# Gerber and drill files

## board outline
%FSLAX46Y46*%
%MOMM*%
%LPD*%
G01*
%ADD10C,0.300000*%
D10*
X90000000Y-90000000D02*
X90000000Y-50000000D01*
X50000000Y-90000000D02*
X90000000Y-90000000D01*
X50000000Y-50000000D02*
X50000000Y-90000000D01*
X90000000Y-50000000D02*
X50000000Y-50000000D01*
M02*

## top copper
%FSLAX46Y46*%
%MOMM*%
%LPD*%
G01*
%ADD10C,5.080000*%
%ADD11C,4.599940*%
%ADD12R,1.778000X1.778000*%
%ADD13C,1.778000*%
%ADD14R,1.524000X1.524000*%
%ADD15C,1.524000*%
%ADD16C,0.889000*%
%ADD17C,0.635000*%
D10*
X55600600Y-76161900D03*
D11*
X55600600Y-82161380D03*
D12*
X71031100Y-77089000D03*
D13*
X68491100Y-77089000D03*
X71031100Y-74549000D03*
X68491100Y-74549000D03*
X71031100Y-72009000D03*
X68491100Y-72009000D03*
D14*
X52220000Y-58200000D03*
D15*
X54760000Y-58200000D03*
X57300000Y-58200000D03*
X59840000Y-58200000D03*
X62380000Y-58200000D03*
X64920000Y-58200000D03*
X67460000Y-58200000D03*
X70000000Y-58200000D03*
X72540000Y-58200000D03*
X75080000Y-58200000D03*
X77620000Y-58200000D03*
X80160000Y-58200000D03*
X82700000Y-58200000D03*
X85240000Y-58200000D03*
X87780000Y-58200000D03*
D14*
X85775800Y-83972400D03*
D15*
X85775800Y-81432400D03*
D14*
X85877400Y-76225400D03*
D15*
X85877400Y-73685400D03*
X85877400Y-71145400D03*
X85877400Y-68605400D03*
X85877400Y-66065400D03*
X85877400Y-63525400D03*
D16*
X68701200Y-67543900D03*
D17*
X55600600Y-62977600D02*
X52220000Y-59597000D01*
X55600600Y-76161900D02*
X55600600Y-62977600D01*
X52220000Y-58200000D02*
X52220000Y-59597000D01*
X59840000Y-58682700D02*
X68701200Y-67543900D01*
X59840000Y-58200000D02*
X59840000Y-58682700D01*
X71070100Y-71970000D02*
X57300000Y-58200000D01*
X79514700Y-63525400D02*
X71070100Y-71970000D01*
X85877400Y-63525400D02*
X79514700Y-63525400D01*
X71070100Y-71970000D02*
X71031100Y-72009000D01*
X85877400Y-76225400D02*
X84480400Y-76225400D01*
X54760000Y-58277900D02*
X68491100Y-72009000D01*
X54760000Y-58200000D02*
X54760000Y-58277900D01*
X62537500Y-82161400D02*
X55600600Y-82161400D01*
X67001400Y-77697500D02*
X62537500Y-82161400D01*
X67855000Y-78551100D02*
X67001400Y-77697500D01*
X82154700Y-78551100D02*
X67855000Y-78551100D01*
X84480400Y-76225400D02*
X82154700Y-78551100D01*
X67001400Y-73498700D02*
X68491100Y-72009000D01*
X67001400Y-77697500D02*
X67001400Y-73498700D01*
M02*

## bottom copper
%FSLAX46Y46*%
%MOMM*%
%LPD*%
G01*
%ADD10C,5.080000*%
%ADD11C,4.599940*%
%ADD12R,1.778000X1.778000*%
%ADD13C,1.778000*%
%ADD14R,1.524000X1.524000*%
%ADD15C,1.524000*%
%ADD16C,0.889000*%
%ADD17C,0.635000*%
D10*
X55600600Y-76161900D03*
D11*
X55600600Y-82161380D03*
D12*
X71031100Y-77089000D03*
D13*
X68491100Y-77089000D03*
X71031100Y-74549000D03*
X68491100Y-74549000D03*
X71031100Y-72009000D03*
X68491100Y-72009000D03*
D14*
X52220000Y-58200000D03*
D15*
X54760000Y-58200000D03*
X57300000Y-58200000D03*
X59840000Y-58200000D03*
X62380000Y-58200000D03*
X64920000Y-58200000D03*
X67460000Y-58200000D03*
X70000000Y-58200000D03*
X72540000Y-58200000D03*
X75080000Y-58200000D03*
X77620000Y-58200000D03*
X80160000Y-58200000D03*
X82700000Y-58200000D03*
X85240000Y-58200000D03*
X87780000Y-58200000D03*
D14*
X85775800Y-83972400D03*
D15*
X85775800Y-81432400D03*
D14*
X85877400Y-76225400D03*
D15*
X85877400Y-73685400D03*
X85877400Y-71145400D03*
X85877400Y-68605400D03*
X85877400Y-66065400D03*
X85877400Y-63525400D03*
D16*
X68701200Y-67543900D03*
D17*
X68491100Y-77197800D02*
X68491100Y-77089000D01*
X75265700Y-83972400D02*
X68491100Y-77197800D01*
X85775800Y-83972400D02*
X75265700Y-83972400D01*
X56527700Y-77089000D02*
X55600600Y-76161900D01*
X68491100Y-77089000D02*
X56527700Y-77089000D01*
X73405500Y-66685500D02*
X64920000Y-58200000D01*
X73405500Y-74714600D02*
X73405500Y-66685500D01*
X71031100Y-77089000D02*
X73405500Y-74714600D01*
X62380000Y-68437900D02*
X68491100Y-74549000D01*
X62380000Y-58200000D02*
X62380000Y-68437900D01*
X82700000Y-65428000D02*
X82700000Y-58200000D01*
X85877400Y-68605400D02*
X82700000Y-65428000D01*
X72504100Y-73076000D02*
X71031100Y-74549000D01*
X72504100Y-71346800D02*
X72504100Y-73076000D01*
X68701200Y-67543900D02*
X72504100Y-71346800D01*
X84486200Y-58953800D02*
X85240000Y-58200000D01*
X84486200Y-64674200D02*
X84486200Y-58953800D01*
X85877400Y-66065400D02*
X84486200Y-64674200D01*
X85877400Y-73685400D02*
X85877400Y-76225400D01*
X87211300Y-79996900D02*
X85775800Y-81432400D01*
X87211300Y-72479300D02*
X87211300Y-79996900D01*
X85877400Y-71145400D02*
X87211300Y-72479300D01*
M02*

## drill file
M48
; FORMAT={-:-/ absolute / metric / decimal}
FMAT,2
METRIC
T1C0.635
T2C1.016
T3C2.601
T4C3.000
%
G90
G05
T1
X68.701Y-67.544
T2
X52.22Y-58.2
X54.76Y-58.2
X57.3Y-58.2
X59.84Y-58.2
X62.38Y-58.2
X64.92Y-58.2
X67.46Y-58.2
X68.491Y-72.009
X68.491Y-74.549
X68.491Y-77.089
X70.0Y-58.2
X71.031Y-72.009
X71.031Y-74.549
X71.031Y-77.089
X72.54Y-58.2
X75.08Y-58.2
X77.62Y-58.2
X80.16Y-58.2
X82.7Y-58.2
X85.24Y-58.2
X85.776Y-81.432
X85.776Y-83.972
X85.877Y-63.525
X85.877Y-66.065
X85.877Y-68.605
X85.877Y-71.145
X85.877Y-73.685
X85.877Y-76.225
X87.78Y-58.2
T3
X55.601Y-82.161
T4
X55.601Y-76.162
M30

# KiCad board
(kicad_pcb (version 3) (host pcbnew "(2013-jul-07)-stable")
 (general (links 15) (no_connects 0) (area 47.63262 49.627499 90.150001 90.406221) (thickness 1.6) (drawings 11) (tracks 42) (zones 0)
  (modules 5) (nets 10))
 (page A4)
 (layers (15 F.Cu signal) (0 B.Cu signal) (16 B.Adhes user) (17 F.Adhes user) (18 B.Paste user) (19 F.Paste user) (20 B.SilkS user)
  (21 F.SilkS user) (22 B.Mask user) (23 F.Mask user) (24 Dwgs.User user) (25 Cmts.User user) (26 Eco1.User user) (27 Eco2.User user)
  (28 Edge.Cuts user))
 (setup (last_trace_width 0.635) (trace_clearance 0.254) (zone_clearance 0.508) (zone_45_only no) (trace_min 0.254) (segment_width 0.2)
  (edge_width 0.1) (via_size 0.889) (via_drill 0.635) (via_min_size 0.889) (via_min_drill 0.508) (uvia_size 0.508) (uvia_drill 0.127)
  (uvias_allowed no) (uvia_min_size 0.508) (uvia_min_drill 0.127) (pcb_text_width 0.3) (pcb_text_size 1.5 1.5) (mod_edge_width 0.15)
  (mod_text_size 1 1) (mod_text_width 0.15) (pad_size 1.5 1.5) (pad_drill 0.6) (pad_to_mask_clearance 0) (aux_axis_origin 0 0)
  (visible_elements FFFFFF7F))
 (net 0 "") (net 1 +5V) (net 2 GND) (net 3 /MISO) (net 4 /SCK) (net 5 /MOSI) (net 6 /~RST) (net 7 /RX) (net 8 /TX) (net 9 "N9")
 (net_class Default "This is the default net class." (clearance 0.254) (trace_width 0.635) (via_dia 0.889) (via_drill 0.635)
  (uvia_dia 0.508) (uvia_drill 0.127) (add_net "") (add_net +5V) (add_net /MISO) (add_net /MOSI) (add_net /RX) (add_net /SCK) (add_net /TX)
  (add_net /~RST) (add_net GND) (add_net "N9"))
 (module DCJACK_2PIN (layer F.Cu) (at 55.6006 76.1619 270)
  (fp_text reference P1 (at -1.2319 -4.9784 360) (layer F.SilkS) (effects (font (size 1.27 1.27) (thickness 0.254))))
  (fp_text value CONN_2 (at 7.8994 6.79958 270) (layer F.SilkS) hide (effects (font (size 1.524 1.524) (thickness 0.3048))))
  (pad 1 thru_hole circle (at 0 0 270) (size 5.08 5.08) (drill 2.99974) (layers *.Cu *.Mask F.SilkS) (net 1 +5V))
  (pad 2 thru_hole circle (at 5.99948 0 270) (size 4.59994 4.59994) (drill 2.60096) (layers *.Cu *.Mask F.SilkS) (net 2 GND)))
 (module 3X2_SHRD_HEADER (layer F.Cu) (at 69.7611 74.549 90)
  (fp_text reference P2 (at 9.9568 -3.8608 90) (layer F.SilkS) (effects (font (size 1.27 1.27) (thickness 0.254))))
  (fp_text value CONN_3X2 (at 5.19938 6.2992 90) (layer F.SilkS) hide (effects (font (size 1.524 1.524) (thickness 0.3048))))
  (pad 1 thru_hole rect (at -2.54 1.27 90) (size 1.778 1.778) (drill 1.016) (layers *.Cu *.Mask F.SilkS) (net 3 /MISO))
  (pad 2 thru_hole circle (at -2.54 -1.27 90) (size 1.778 1.778) (drill 1.016) (layers *.Cu *.Mask F.SilkS) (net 1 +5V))
  (pad 3 thru_hole circle (at 0 1.27 90) (size 1.778 1.778) (drill 1.016) (layers *.Cu *.Mask F.SilkS) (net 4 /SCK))
  (pad 4 thru_hole circle (at 0 -1.27 90) (size 1.778 1.778) (drill 1.016) (layers *.Cu *.Mask F.SilkS) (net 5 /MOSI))
  (pad 5 thru_hole circle (at 2.54 1.27 90) (size 1.778 1.778) (drill 1.016) (layers *.Cu *.Mask F.SilkS) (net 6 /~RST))
  (pad 6 thru_hole circle (at 2.54 -1.27 90) (size 1.778 1.778) (drill 1.016) (layers *.Cu *.Mask F.SilkS) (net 2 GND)))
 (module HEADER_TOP (layer F.Cu) (at 70 58.2)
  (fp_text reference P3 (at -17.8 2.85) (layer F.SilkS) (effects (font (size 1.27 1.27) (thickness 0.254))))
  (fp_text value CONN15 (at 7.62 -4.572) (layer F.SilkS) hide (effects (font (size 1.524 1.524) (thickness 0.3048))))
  (pad 1 thru_hole rect (at -17.78 0) (size 1.524 1.524) (drill 1.016) (layers *.Cu *.Mask F.SilkS) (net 1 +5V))
  (pad 2 thru_hole circle (at -15.24 0) (size 1.524 1.524) (drill 1.016) (layers *.Cu *.Mask F.SilkS) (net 2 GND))
  (pad 3 thru_hole circle (at -12.7 0) (size 1.524 1.524) (drill 1.016) (layers *.Cu *.Mask F.SilkS) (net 6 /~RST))
  (pad 4 thru_hole circle (at -10.16 0) (size 1.524 1.524) (drill 1.016) (layers *.Cu *.Mask F.SilkS) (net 4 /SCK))
  (pad 5 thru_hole circle (at -7.62 0) (size 1.524 1.524) (drill 1.016) (layers *.Cu *.Mask F.SilkS) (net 5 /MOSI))
  (pad 6 thru_hole circle (at -5.08 0) (size 1.524 1.524) (drill 1.016) (layers *.Cu *.Mask F.SilkS) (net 3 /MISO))
  (pad 7 thru_hole circle (at -2.54 0) (size 1.524 1.524) (drill 1.016) (layers *.Cu *.Mask F.SilkS))
  (pad 8 thru_hole circle (at 0 0) (size 1.524 1.524) (drill 1.016) (layers *.Cu *.Mask F.SilkS))
  (pad 9 thru_hole circle (at 2.54 0) (size 1.524 1.524) (drill 1.016) (layers *.Cu *.Mask F.SilkS))
  (pad 10 thru_hole circle (at 5.08 0) (size 1.524 1.524) (drill 1.016) (layers *.Cu *.Mask F.SilkS))
  (pad 11 thru_hole circle (at 7.62 0) (size 1.524 1.524) (drill 1.016) (layers *.Cu *.Mask F.SilkS))
  (pad 12 thru_hole circle (at 10.16 0) (size 1.524 1.524) (drill 1.016) (layers *.Cu *.Mask F.SilkS))
  (pad 13 thru_hole circle (at 12.7 0) (size 1.524 1.524) (drill 1.016) (layers *.Cu *.Mask F.SilkS) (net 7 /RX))
  (pad 14 thru_hole circle (at 15.24 0) (size 1.524 1.524) (drill 1.016) (layers *.Cu *.Mask F.SilkS) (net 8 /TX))
  (pad 15 thru_hole circle (at 17.78 0) (size 1.524 1.524) (drill 1.016) (layers *.Cu *.Mask F.SilkS)))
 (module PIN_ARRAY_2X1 (layer F.Cu) (at 85.7758 82.7024 90)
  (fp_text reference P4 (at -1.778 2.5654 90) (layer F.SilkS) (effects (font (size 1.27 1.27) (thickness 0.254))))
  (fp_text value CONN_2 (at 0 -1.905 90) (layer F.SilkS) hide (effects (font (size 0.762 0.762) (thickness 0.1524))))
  (pad 1 thru_hole rect (at -1.27 0 90) (size 1.524 1.524) (drill 1.016) (layers *.Cu *.Mask F.SilkS) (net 1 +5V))
  (pad 2 thru_hole circle (at 1.27 0 90) (size 1.524 1.524) (drill 1.016) (layers *.Cu *.Mask F.SilkS) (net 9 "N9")))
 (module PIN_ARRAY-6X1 (layer F.Cu) (at 85.8774 69.8754 90)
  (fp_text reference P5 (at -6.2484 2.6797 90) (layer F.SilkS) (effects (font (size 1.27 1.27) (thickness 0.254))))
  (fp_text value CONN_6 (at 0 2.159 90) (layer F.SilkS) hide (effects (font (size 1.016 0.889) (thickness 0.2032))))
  (pad 1 thru_hole rect (at -6.35 0 90) (size 1.524 1.524) (drill 1.016) (layers *.Cu *.Mask F.SilkS) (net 2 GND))
  (pad 2 thru_hole circle (at -3.81 0 90) (size 1.524 1.524) (drill 1.016) (layers *.Cu *.Mask F.SilkS) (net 2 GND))
  (pad 3 thru_hole circle (at -1.27 0 90) (size 1.524 1.524) (drill 1.016) (layers *.Cu *.Mask F.SilkS) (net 9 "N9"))
  (pad 4 thru_hole circle (at 1.27 0 90) (size 1.524 1.524) (drill 1.016) (layers *.Cu *.Mask F.SilkS) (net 7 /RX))
  (pad 5 thru_hole circle (at 3.81 0 90) (size 1.524 1.524) (drill 1.016) (layers *.Cu *.Mask F.SilkS) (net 8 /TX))
  (pad 6 thru_hole circle (at 6.35 0 90) (size 1.524 1.524) (drill 1.016) (layers *.Cu *.Mask F.SilkS) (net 6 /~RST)))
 (gr_line (start 90 90) (end 90 50) (angle 90) (layer Edge.Cuts) (width 0.3))
 (gr_line (start 50 90) (end 90 90) (angle 90) (layer Edge.Cuts) (width 0.3))
 (gr_line (start 50 50) (end 50 90) (angle 90) (layer Edge.Cuts) (width 0.3))
 (gr_line (start 90 50) (end 50 50) (angle 90) (layer Edge.Cuts) (width 0.3))
 (segment (start 55.6006 62.9776) (end 52.22 59.597) (width 0.635) (layer F.Cu) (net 1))
 (segment (start 55.6006 76.1619) (end 55.6006 62.9776) (width 0.635) (layer F.Cu) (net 1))
 (segment (start 52.22 58.2) (end 52.22 59.597) (width 0.635) (layer F.Cu) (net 1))
 (segment (start 68.4911 77.1978) (end 68.4911 77.089) (width 0.635) (layer B.Cu) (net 1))
 (segment (start 75.2657 83.9724) (end 68.4911 77.1978) (width 0.635) (layer B.Cu) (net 1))
 (segment (start 85.7758 83.9724) (end 75.2657 83.9724) (width 0.635) (layer B.Cu) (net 1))
 (segment (start 56.5277 77.089) (end 55.6006 76.1619) (width 0.635) (layer B.Cu) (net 1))
 (segment (start 68.4911 77.089) (end 56.5277 77.089) (width 0.635) (layer B.Cu) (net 1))
 (segment (start 73.4055 66.6855) (end 64.92 58.2) (width 0.635) (layer B.Cu) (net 3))
 (segment (start 73.4055 74.7146) (end 73.4055 66.6855) (width 0.635) (layer B.Cu) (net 3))
 (segment (start 71.0311 77.089) (end 73.4055 74.7146) (width 0.635) (layer B.Cu) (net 3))
 (segment (start 62.38 68.4379) (end 68.4911 74.549) (width 0.635) (layer B.Cu) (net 5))
 (segment (start 62.38 58.2) (end 62.38 68.4379) (width 0.635) (layer B.Cu) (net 5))
 (segment (start 82.7 65.428) (end 82.7 58.2) (width 0.635) (layer B.Cu) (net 7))
 (segment (start 85.8774 68.6054) (end 82.7 65.428) (width 0.635) (layer B.Cu) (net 7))
 (via (at 68.7012 67.5439) (size 0.889) (layers F.Cu B.Cu) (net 4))
 (segment (start 72.5041 73.076) (end 71.0311 74.549) (width 0.635) (layer B.Cu) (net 4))
 (segment (start 72.5041 71.3468) (end 72.5041 73.076) (width 0.635) (layer B.Cu) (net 4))
 (segment (start 68.7012 67.5439) (end 72.5041 71.3468) (width 0.635) (layer B.Cu) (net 4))
 (segment (start 59.84 58.6827) (end 68.7012 67.5439) (width 0.635) (layer F.Cu) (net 4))
 (segment (start 59.84 58.2) (end 59.84 58.6827) (width 0.635) (layer F.Cu) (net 4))
 (segment (start 84.4862 58.9538) (end 85.24 58.2) (width 0.635) (layer B.Cu) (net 8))
 (segment (start 84.4862 64.6742) (end 84.4862 58.9538) (width 0.635) (layer B.Cu) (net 8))
 (segment (start 85.8774 66.0654) (end 84.4862 64.6742) (width 0.635) (layer B.Cu) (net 8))
 (segment (start 71.0701 71.97) (end 57.3 58.2) (width 0.635) (layer F.Cu) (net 6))
 (segment (start 79.5147 63.5254) (end 71.0701 71.97) (width 0.635) (layer F.Cu) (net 6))
 (segment (start 85.8774 63.5254) (end 79.5147 63.5254) (width 0.635) (layer F.Cu) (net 6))
 (segment (start 71.0701 71.97) (end 71.0311 72.009) (width 0.635) (layer F.Cu) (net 6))
 (segment (start 85.8774 73.6854) (end 85.8774 76.2254) (width 0.635) (layer B.Cu) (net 2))
 (segment (start 85.8774 76.2254) (end 84.4804 76.2254) (width 0.635) (layer F.Cu) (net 2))
 (segment (start 54.76 58.2779) (end 68.4911 72.009) (width 0.635) (layer F.Cu) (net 2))
 (segment (start 54.76 58.2) (end 54.76 58.2779) (width 0.635) (layer F.Cu) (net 2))
 (segment (start 62.5375 82.1614) (end 55.6006 82.1614) (width 0.635) (layer F.Cu) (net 2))
 (segment (start 67.0014 77.6975) (end 62.5375 82.1614) (width 0.635) (layer F.Cu) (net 2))
 (segment (start 67.855 78.5511) (end 67.0014 77.6975) (width 0.635) (layer F.Cu) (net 2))
 (segment (start 82.1547 78.5511) (end 67.855 78.5511) (width 0.635) (layer F.Cu) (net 2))
 (segment (start 84.4804 76.2254) (end 82.1547 78.5511) (width 0.635) (layer F.Cu) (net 2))
 (segment (start 67.0014 73.4987) (end 68.4911 72.009) (width 0.635) (layer F.Cu) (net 2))
 (segment (start 67.0014 77.6975) (end 67.0014 73.4987) (width 0.635) (layer F.Cu) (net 2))
 (segment (start 87.2113 79.9969) (end 85.7758 81.4324) (width 0.635) (layer B.Cu) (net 9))
 (segment (start 87.2113 72.4793) (end 87.2113 79.9969) (width 0.635) (layer B.Cu) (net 9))
 (segment (start 85.8774 71.1454) (end 87.2113 72.4793) (width 0.635) (layer B.Cu) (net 9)))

